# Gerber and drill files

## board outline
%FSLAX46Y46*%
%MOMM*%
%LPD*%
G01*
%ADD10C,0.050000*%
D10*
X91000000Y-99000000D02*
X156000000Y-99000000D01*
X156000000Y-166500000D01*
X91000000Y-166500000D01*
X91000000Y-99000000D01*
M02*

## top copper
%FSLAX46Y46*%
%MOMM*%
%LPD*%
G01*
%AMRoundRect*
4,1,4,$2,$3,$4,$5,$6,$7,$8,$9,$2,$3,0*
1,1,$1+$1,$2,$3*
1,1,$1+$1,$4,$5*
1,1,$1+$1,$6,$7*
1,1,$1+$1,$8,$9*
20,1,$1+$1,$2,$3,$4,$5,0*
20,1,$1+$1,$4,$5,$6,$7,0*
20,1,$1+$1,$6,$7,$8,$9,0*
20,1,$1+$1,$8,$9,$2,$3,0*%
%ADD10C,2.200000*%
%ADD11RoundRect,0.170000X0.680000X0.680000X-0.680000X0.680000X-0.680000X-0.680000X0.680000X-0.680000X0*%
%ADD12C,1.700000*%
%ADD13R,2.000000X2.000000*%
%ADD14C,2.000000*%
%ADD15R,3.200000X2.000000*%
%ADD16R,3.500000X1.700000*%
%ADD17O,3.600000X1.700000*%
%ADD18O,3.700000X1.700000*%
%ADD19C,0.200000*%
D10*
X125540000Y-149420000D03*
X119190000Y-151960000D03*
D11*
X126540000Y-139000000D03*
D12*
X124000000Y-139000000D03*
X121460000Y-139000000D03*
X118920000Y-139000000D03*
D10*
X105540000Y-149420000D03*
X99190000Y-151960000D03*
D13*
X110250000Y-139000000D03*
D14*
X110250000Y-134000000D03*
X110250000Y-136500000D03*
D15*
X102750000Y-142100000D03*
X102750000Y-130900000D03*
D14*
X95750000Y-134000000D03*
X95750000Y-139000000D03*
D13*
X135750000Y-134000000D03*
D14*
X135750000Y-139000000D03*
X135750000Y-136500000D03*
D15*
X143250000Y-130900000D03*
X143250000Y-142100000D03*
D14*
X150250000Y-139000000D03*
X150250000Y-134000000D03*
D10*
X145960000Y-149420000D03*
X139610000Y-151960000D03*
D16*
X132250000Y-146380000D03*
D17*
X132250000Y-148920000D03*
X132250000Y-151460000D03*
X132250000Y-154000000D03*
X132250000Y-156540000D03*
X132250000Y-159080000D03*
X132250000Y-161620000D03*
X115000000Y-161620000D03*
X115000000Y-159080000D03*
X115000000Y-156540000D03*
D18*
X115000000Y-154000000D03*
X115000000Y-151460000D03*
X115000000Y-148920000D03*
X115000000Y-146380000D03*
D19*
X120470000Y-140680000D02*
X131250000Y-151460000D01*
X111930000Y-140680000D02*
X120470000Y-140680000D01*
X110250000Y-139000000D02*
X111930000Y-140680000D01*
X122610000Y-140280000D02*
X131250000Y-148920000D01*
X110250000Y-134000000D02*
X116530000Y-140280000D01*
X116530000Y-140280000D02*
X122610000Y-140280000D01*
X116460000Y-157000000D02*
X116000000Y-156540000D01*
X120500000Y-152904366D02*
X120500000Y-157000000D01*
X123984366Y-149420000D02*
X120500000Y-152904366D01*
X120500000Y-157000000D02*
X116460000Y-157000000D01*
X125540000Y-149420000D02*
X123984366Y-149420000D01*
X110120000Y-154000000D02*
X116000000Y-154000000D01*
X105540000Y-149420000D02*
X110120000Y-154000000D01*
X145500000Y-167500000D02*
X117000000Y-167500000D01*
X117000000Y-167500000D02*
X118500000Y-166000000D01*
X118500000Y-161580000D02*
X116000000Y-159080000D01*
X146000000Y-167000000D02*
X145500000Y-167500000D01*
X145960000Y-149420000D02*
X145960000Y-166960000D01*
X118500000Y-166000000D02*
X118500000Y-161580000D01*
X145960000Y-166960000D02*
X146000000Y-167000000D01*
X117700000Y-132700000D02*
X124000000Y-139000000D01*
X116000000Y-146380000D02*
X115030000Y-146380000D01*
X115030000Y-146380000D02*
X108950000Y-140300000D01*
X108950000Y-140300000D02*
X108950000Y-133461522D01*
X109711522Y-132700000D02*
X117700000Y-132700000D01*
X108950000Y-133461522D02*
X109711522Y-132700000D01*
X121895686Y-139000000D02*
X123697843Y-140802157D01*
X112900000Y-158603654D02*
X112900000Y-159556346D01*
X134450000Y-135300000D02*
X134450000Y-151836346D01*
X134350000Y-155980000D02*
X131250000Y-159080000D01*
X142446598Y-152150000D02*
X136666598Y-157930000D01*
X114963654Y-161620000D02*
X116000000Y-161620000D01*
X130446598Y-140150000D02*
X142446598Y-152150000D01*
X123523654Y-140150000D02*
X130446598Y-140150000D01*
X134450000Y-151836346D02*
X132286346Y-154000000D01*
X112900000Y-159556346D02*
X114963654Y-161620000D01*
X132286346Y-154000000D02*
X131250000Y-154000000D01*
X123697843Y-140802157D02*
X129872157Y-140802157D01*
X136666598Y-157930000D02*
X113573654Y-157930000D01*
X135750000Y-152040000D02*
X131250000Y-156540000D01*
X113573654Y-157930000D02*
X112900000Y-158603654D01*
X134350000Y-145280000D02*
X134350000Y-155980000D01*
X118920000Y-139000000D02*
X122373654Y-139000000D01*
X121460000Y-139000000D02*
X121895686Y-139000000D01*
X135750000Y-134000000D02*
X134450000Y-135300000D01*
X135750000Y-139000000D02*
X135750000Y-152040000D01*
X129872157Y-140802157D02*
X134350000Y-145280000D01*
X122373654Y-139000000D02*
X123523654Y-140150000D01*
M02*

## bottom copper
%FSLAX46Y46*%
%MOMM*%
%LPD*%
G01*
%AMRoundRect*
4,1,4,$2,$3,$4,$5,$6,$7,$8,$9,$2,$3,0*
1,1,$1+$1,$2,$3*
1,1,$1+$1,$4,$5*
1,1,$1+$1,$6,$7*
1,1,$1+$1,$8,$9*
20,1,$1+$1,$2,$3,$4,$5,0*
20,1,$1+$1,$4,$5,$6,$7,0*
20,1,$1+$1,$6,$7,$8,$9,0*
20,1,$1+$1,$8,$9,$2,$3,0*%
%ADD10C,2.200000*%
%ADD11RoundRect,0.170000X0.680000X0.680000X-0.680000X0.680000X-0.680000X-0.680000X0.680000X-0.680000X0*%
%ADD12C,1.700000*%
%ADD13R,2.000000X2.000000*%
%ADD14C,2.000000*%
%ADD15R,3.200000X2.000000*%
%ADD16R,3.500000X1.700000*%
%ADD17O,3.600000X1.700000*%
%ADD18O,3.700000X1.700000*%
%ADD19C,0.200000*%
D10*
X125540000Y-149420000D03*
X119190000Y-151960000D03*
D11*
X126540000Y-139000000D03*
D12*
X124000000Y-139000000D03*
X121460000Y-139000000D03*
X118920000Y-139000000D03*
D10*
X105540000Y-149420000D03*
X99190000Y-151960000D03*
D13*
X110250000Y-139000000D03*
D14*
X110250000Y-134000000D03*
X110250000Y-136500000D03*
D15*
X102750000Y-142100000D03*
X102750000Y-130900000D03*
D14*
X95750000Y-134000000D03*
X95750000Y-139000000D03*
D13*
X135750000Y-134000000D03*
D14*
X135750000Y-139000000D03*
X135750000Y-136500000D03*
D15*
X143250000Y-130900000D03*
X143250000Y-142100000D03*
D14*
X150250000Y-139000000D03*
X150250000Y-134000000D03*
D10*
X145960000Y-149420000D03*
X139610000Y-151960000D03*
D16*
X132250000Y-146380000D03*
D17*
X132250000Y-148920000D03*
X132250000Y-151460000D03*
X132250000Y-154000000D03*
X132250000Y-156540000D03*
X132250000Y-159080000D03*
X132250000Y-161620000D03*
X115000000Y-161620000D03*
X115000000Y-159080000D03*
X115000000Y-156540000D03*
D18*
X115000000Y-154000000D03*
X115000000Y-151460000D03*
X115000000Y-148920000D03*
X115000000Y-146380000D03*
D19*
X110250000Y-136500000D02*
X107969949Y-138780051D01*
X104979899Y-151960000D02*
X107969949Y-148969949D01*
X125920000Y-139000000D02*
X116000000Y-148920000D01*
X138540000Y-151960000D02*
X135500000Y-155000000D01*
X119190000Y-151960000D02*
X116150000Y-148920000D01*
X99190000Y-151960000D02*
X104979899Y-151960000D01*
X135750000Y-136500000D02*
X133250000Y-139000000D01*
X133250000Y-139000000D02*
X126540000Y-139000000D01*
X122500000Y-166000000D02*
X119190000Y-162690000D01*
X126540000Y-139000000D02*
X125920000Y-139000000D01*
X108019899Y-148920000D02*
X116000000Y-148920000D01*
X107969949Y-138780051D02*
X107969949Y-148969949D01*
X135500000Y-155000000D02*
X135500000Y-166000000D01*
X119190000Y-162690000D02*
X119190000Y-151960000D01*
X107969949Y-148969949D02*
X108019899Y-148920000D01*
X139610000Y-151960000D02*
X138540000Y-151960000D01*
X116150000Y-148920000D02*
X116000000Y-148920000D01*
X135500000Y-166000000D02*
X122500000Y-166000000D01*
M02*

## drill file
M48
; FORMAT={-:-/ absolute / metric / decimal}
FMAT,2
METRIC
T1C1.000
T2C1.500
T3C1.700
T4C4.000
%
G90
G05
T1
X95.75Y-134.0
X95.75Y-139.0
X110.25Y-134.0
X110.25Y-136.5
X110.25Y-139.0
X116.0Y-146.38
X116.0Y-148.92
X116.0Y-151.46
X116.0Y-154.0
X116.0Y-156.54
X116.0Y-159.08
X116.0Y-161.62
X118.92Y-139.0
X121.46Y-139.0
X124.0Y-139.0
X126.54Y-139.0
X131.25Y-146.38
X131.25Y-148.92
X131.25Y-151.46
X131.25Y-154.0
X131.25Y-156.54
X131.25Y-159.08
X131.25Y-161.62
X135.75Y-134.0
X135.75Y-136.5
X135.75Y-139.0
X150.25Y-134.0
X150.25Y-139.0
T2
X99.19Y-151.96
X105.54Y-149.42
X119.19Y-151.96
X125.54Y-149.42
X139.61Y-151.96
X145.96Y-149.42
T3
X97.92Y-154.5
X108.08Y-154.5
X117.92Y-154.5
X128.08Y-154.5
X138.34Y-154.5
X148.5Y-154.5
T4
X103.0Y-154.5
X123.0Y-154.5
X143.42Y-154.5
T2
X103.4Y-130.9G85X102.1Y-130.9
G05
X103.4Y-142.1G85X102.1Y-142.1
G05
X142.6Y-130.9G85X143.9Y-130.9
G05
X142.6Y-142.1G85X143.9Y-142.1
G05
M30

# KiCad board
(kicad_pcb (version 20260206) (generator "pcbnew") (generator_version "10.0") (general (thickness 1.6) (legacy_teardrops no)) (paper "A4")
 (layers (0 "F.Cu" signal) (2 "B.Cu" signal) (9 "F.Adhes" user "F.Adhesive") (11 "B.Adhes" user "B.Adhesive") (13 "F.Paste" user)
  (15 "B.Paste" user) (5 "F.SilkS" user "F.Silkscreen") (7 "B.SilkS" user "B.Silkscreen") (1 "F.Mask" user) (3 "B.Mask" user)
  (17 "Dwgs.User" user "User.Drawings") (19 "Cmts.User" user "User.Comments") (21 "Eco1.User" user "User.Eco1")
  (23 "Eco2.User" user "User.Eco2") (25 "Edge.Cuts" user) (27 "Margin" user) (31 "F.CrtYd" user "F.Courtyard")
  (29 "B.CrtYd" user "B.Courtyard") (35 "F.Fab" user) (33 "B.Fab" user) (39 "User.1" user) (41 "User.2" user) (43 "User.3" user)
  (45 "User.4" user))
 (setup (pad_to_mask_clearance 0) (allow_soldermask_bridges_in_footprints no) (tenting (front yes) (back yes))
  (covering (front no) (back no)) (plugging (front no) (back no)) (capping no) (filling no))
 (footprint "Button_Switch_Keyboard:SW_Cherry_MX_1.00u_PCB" (layer "F.Cu") (at 125.54 149.42)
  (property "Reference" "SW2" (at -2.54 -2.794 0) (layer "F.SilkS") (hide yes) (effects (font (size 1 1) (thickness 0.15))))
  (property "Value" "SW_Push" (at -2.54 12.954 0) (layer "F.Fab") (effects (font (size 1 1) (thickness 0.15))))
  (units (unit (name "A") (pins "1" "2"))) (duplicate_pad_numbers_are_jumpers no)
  (pad "" np_thru_hole circle (at -7.62 5.08) (size 1.7 1.7) (drill 1.7) (layers "*.Cu" "*.Mask"))
  (pad "" np_thru_hole circle (at -2.54 5.08) (size 4 4) (drill 4) (layers "*.Cu" "*.Mask"))
  (pad "" np_thru_hole circle (at 2.54 5.08) (size 1.7 1.7) (drill 1.7) (layers "*.Cu" "*.Mask"))
  (pad "1" thru_hole circle (at 0 0) (size 2.2 2.2) (drill 1.5) (layers "*.Cu" "*.Mask") (remove_unused_layers no)
   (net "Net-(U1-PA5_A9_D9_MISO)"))
  (pad "2" thru_hole circle (at -6.35 2.54) (size 2.2 2.2) (drill 1.5) (layers "*.Cu" "*.Mask") (remove_unused_layers no) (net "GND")))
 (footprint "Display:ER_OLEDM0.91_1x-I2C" (layer "F.Cu") (at 126.54 139 180)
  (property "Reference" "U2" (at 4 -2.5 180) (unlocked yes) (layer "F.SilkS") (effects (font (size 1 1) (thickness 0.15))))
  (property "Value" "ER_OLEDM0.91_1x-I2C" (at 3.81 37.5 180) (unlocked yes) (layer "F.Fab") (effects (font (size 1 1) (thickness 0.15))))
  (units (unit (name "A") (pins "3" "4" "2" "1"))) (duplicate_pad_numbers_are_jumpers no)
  (pad "1" thru_hole roundrect (at 0 0 180) (size 1.7 1.7) (drill 1) (layers "*.Cu" "*.Mask") (remove_unused_layers no)
   (roundrect_rratio 0.1) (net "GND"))
  (pad "2" thru_hole circle (at 2.54 0 180) (size 1.7 1.7) (drill 1) (layers "*.Cu" "*.Mask") (remove_unused_layers no)
   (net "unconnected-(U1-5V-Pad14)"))
  (pad "3" thru_hole circle (at 5.08 0 180) (size 1.7 1.7) (drill 1) (layers "*.Cu" "*.Mask") (remove_unused_layers no)
   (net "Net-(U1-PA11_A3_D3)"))
  (pad "4" thru_hole circle (at 7.62 0 180) (size 1.7 1.7) (drill 1) (layers "*.Cu" "*.Mask") (remove_unused_layers no)
   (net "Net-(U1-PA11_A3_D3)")))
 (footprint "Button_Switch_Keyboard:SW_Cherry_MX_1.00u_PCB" (layer "F.Cu") (at 105.54 149.42)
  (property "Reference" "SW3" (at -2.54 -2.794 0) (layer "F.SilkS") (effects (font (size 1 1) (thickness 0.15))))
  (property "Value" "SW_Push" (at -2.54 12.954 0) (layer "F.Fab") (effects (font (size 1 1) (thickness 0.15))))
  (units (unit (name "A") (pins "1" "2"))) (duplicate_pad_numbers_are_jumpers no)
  (pad "" np_thru_hole circle (at -7.62 5.08) (size 1.7 1.7) (drill 1.7) (layers "*.Cu" "*.Mask"))
  (pad "" np_thru_hole circle (at -2.54 5.08) (size 4 4) (drill 4) (layers "*.Cu" "*.Mask"))
  (pad "" np_thru_hole circle (at 2.54 5.08) (size 1.7 1.7) (drill 1.7) (layers "*.Cu" "*.Mask"))
  (pad "1" thru_hole circle (at 0 0) (size 2.2 2.2) (drill 1.5) (layers "*.Cu" "*.Mask") (remove_unused_layers no)
   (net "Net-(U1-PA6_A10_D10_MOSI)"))
  (pad "2" thru_hole circle (at -6.35 2.54) (size 2.2 2.2) (drill 1.5) (layers "*.Cu" "*.Mask") (remove_unused_layers no) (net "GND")))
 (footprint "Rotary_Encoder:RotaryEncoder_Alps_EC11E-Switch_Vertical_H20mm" (layer "F.Cu") (at 110.25 139 180)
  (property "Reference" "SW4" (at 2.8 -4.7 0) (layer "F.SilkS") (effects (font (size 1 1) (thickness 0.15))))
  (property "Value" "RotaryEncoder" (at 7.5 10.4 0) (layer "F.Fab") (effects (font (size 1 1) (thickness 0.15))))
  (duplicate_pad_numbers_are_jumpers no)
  (pad "A" thru_hole rect (at 0 0 180) (size 2 2) (drill 1) (layers "*.Cu" "*.Mask") (remove_unused_layers no) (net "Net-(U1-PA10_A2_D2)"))
  (pad "B" thru_hole circle (at 0 5 180) (size 2 2) (drill 1) (layers "*.Cu" "*.Mask") (remove_unused_layers no) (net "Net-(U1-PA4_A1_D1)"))
  (pad "C" thru_hole circle (at 0 2.5 180) (size 2 2) (drill 1) (layers "*.Cu" "*.Mask") (remove_unused_layers no) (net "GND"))
  (pad "MP" thru_hole rect (at 7.5 -3.1 180) (size 3.2 2) (drill oval 2.8 1.5) (layers "*.Cu" "*.Mask") (remove_unused_layers no))
  (pad "MP" thru_hole rect (at 7.5 8.1 180) (size 3.2 2) (drill oval 2.8 1.5) (layers "*.Cu" "*.Mask") (remove_unused_layers no))
  (pad "S1" thru_hole circle (at 14.5 5 180) (size 2 2) (drill 1) (layers "*.Cu" "*.Mask") (remove_unused_layers no))
  (pad "S2" thru_hole circle (at 14.5 0 180) (size 2 2) (drill 1) (layers "*.Cu" "*.Mask") (remove_unused_layers no)))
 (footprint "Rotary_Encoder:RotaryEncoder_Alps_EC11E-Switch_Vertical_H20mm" (layer "F.Cu") (at 135.75 134)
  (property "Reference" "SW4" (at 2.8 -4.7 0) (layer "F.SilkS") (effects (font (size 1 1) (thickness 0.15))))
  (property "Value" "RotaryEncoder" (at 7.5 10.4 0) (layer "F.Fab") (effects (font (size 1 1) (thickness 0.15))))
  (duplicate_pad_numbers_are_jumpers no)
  (pad "A" thru_hole rect (at 0 0) (size 2 2) (drill 1) (layers "*.Cu" "*.Mask") (remove_unused_layers no) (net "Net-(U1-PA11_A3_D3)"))
  (pad "B" thru_hole circle (at 0 5) (size 2 2) (drill 1) (layers "*.Cu" "*.Mask") (remove_unused_layers no) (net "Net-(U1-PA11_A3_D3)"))
  (pad "C" thru_hole circle (at 0 2.5) (size 2 2) (drill 1) (layers "*.Cu" "*.Mask") (remove_unused_layers no) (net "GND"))
  (pad "MP" thru_hole rect (at 7.5 -3.1) (size 3.2 2) (drill oval 2.8 1.5) (layers "*.Cu" "*.Mask") (remove_unused_layers no))
  (pad "MP" thru_hole rect (at 7.5 8.1) (size 3.2 2) (drill oval 2.8 1.5) (layers "*.Cu" "*.Mask") (remove_unused_layers no))
  (pad "S1" thru_hole circle (at 14.5 5) (size 2 2) (drill 1) (layers "*.Cu" "*.Mask") (remove_unused_layers no))
  (pad "S2" thru_hole circle (at 14.5 0) (size 2 2) (drill 1) (layers "*.Cu" "*.Mask") (remove_unused_layers no)))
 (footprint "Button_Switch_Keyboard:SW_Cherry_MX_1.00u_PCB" (layer "F.Cu") (at 145.96 149.42)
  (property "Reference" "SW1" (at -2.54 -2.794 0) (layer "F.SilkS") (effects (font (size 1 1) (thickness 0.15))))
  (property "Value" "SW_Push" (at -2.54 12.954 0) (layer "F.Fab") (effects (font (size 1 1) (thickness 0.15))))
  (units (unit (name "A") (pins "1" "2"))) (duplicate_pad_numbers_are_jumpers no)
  (pad "" np_thru_hole circle (at -7.62 5.08) (size 1.7 1.7) (drill 1.7) (layers "*.Cu" "*.Mask"))
  (pad "" np_thru_hole circle (at -2.54 5.08) (size 4 4) (drill 4) (layers "*.Cu" "*.Mask"))
  (pad "" np_thru_hole circle (at 2.54 5.08) (size 1.7 1.7) (drill 1.7) (layers "*.Cu" "*.Mask"))
  (pad "1" thru_hole circle (at 0 0) (size 2.2 2.2) (drill 1.5) (layers "*.Cu" "*.Mask") (remove_unused_layers no)
   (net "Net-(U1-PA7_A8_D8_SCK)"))
  (pad "2" thru_hole circle (at -6.35 2.54) (size 2.2 2.2) (drill 1.5) (layers "*.Cu" "*.Mask") (remove_unused_layers no) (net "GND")))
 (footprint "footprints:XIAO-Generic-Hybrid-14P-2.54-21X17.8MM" (layer "B.Cu") (at 123.625 154 180)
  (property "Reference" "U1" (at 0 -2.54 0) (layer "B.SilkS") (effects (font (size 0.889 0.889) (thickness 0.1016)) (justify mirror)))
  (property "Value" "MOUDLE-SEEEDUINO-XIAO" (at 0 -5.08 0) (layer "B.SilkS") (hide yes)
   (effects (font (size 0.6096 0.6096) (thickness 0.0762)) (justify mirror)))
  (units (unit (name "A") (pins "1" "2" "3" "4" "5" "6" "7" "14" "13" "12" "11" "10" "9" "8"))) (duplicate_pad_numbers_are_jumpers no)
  (pad "1" thru_hole rect (at -7.625 7.62 180) (size 3.5 1.7) (drill 1 (offset -1 0)) (layers "*.Cu" "*.Mask") (remove_unused_layers no)
   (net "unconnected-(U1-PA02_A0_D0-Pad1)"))
  (pad "2" thru_hole oval (at -7.625 5.08 180) (size 3.6 1.7) (drill 1 (offset -1 0)) (layers "*.Cu" "*.Mask") (remove_unused_layers no)
   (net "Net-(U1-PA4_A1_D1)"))
  (pad "3" thru_hole oval (at -7.625 2.54 180) (size 3.6 1.7) (drill 1 (offset -1 0)) (layers "*.Cu" "*.Mask") (remove_unused_layers no)
   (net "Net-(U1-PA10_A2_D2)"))
  (pad "4" thru_hole oval (at -7.625 0 180) (size 3.6 1.7) (drill 1 (offset -1 0)) (layers "*.Cu" "*.Mask") (remove_unused_layers no)
   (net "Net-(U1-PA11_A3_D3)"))
  (pad "5" thru_hole oval (at -7.625 -2.54 180) (size 3.6 1.7) (drill 1 (offset -1 0)) (layers "*.Cu" "*.Mask") (remove_unused_layers no)
   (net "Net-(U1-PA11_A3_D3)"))
  (pad "6" thru_hole oval (at -7.625 -5.08) (size 3.6 1.7) (drill 1 (offset 1 0)) (layers "*.Cu" "*.Mask") (remove_unused_layers no)
   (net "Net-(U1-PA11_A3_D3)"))
  (pad "7" thru_hole oval (at -7.625 -7.62 180) (size 3.6 1.7) (drill 1 (offset -1 0)) (layers "*.Cu" "*.Mask") (remove_unused_layers no)
   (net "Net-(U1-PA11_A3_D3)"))
  (pad "8" thru_hole oval (at 7.625 -7.62 180) (size 3.6 1.7) (drill 1 (offset 1 0)) (layers "*.Cu" "*.Mask") (remove_unused_layers no)
   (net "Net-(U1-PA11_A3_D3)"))
  (pad "9" thru_hole oval (at 7.625 -5.08 180) (size 3.6 1.7) (drill 1 (offset 1 0)) (layers "*.Cu" "*.Mask") (remove_unused_layers no)
   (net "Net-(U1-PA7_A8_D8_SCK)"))
  (pad "10" thru_hole oval (at 7.625 -2.54 180) (size 3.6 1.7) (drill 1 (offset 1 0)) (layers "*.Cu" "*.Mask") (remove_unused_layers no)
   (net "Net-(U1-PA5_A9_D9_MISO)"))
  (pad "11" thru_hole oval (at 7.625 0 180) (size 3.7 1.7) (drill 1 (offset 1 0)) (layers "*.Cu" "*.Mask") (remove_unused_layers no)
   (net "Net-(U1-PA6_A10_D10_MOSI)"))
  (pad "12" thru_hole oval (at 7.625 2.54 180) (size 3.7 1.7) (drill 1 (offset 1 0)) (layers "*.Cu" "*.Mask") (remove_unused_layers no)
   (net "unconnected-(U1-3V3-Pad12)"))
  (pad "13" thru_hole oval (at 7.625 5.08 180) (size 3.7 1.7) (drill 1 (offset 1 0)) (layers "*.Cu" "*.Mask") (remove_unused_layers no)
   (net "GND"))
  (pad "14" thru_hole oval (at 7.625 7.62 180) (size 3.7 1.7) (drill 1 (offset 1 0)) (layers "*.Cu" "*.Mask") (remove_unused_layers no)
   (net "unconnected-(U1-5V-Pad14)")))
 (gr_rect (start 91 99) (end 156 166.5) (stroke (width 0.05) (type default)) (fill no) (layer "Edge.Cuts"))
 (segment (start 120.47 140.68) (end 131.25 151.46) (width 0.2) (layer "F.Cu") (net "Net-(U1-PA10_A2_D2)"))
 (segment (start 111.93 140.68) (end 120.47 140.68) (width 0.2) (layer "F.Cu") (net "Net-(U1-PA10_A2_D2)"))
 (segment (start 110.25 139) (end 111.93 140.68) (width 0.2) (layer "F.Cu") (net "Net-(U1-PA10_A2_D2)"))
 (segment (start 122.61 140.28) (end 131.25 148.92) (width 0.2) (layer "F.Cu") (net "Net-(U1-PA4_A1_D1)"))
 (segment (start 110.25 134) (end 116.53 140.28) (width 0.2) (layer "F.Cu") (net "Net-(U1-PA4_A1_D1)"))
 (segment (start 116.53 140.28) (end 122.61 140.28) (width 0.2) (layer "F.Cu") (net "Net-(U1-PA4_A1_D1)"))
 (segment (start 110.25 136.5) (end 107.969949 138.780051) (width 0.2) (layer "B.Cu") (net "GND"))
 (segment (start 104.979899 151.96) (end 107.969949 148.969949) (width 0.2) (layer "B.Cu") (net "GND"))
 (segment (start 125.92 139) (end 116 148.92) (width 0.2) (layer "B.Cu") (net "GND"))
 (segment (start 138.54 151.96) (end 135.5 155) (width 0.2) (layer "B.Cu") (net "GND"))
 (segment (start 119.19 151.96) (end 116.15 148.92) (width 0.2) (layer "B.Cu") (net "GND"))
 (segment (start 99.19 151.96) (end 104.979899 151.96) (width 0.2) (layer "B.Cu") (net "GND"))
 (segment (start 135.75 136.5) (end 133.25 139) (width 0.2) (layer "B.Cu") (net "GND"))
 (segment (start 133.25 139) (end 126.54 139) (width 0.2) (layer "B.Cu") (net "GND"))
 (segment (start 122.5 166) (end 119.19 162.69) (width 0.2) (layer "B.Cu") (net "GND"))
 (segment (start 126.54 139) (end 125.92 139) (width 0.2) (layer "B.Cu") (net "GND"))
 (segment (start 108.019899 148.92) (end 116 148.92) (width 0.2) (layer "B.Cu") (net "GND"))
 (segment (start 107.969949 138.780051) (end 107.969949 148.969949) (width 0.2) (layer "B.Cu") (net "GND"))
 (segment (start 135.5 155) (end 135.5 166) (width 0.2) (layer "B.Cu") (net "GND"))
 (segment (start 119.19 162.69) (end 119.19 151.96) (width 0.2) (layer "B.Cu") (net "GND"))
 (segment (start 107.969949 148.969949) (end 108.019899 148.92) (width 0.2) (layer "B.Cu") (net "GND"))
 (segment (start 139.61 151.96) (end 138.54 151.96) (width 0.2) (layer "B.Cu") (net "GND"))
 (segment (start 116.15 148.92) (end 116 148.92) (width 0.2) (layer "B.Cu") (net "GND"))
 (segment (start 135.5 166) (end 122.5 166) (width 0.2) (layer "B.Cu") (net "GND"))
 (segment (start 116.46 157) (end 116 156.54) (width 0.2) (layer "F.Cu") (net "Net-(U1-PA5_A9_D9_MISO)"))
 (segment (start 120.5 152.904366) (end 120.5 157) (width 0.2) (layer "F.Cu") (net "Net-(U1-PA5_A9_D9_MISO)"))
 (segment (start 123.984366 149.42) (end 120.5 152.904366) (width 0.2) (layer "F.Cu") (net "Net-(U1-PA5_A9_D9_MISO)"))
 (segment (start 120.5 157) (end 116.46 157) (width 0.2) (layer "F.Cu") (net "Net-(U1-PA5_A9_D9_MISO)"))
 (segment (start 125.54 149.42) (end 123.984366 149.42) (width 0.2) (layer "F.Cu") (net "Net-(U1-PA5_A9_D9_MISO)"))
 (segment (start 110.12 154) (end 116 154) (width 0.2) (layer "F.Cu") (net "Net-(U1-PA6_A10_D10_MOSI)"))
 (segment (start 105.54 149.42) (end 110.12 154) (width 0.2) (layer "F.Cu") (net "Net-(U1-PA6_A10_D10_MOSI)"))
 (segment (start 145.5 167.5) (end 117 167.5) (width 0.2) (layer "F.Cu") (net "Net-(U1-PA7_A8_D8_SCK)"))
 (segment (start 117 167.5) (end 118.5 166) (width 0.2) (layer "F.Cu") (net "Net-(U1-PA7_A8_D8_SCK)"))
 (segment (start 118.5 161.58) (end 116 159.08) (width 0.2) (layer "F.Cu") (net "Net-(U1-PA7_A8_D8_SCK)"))
 (segment (start 146 167) (end 145.5 167.5) (width 0.2) (layer "F.Cu") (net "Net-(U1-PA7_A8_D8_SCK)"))
 (segment (start 145.96 149.42) (end 145.96 166.96) (width 0.2) (layer "F.Cu") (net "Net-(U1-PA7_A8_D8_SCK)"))
 (segment (start 118.5 166) (end 118.5 161.58) (width 0.2) (layer "F.Cu") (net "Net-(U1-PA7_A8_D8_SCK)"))
 (segment (start 145.96 166.96) (end 146 167) (width 0.2) (layer "F.Cu") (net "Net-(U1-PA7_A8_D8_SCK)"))
 (segment (start 117.7 132.7) (end 124 139) (width 0.2) (layer "F.Cu") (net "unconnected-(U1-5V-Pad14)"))
 (segment (start 116 146.38) (end 115.03 146.38) (width 0.2) (layer "F.Cu") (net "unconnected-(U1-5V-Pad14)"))
 (segment (start 115.03 146.38) (end 108.95 140.3) (width 0.2) (layer "F.Cu") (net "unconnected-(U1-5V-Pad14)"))
 (segment (start 108.95 140.3) (end 108.95 133.461522) (width 0.2) (layer "F.Cu") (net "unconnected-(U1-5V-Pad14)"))
 (segment (start 109.711522 132.7) (end 117.7 132.7) (width 0.2) (layer "F.Cu") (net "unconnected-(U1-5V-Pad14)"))
 (segment (start 108.95 133.461522) (end 109.711522 132.7) (width 0.2) (layer "F.Cu") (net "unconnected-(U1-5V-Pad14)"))
 (segment (start 121.895686 139) (end 123.697843 140.802157) (width 0.2) (layer "F.Cu") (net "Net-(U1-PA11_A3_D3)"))
 (segment (start 112.9 158.603654) (end 112.9 159.556346) (width 0.2) (layer "F.Cu") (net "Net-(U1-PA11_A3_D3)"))
 (segment (start 134.45 135.3) (end 134.45 151.836346) (width 0.2) (layer "F.Cu") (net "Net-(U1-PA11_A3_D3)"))
 (segment (start 134.35 155.98) (end 131.25 159.08) (width 0.2) (layer "F.Cu") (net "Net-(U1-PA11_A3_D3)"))
 (segment (start 142.446598 152.15) (end 136.666598 157.93) (width 0.2) (layer "F.Cu") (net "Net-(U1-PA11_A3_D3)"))
 (segment (start 114.963654 161.62) (end 116 161.62) (width 0.2) (layer "F.Cu") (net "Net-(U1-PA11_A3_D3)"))
 (segment (start 130.446598 140.15) (end 142.446598 152.15) (width 0.2) (layer "F.Cu") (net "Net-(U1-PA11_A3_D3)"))
 (segment (start 123.523654 140.15) (end 130.446598 140.15) (width 0.2) (layer "F.Cu") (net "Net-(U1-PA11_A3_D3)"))
 (segment (start 134.45 151.836346) (end 132.286346 154) (width 0.2) (layer "F.Cu") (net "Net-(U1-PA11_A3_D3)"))
 (segment (start 112.9 159.556346) (end 114.963654 161.62) (width 0.2) (layer "F.Cu") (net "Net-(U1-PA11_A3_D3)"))
 (segment (start 132.286346 154) (end 131.25 154) (width 0.2) (layer "F.Cu") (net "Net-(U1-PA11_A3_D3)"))
 (segment (start 123.697843 140.802157) (end 129.872157 140.802157) (width 0.2) (layer "F.Cu") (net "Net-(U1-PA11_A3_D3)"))
 (segment (start 136.666598 157.93) (end 113.573654 157.93) (width 0.2) (layer "F.Cu") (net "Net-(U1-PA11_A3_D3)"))
 (segment (start 135.75 152.04) (end 131.25 156.54) (width 0.2) (layer "F.Cu") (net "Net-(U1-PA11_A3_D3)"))
 (segment (start 113.573654 157.93) (end 112.9 158.603654) (width 0.2) (layer "F.Cu") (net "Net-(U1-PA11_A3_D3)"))
 (segment (start 134.35 145.28) (end 134.35 155.98) (width 0.2) (layer "F.Cu") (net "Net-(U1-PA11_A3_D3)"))
 (segment (start 118.92 139) (end 122.373654 139) (width 0.2) (layer "F.Cu") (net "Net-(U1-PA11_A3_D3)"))
 (segment (start 121.46 139) (end 121.895686 139) (width 0.2) (layer "F.Cu") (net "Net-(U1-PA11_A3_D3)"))
 (segment (start 135.75 134) (end 134.45 135.3) (width 0.2) (layer "F.Cu") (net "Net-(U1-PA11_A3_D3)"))
 (segment (start 135.75 139) (end 135.75 152.04) (width 0.2) (layer "F.Cu") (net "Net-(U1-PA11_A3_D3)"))
 (segment (start 129.872157 140.802157) (end 134.35 145.28) (width 0.2) (layer "F.Cu") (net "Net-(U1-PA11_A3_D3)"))
 (segment (start 122.373654 139) (end 123.523654 140.15) (width 0.2) (layer "F.Cu") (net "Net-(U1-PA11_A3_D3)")))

